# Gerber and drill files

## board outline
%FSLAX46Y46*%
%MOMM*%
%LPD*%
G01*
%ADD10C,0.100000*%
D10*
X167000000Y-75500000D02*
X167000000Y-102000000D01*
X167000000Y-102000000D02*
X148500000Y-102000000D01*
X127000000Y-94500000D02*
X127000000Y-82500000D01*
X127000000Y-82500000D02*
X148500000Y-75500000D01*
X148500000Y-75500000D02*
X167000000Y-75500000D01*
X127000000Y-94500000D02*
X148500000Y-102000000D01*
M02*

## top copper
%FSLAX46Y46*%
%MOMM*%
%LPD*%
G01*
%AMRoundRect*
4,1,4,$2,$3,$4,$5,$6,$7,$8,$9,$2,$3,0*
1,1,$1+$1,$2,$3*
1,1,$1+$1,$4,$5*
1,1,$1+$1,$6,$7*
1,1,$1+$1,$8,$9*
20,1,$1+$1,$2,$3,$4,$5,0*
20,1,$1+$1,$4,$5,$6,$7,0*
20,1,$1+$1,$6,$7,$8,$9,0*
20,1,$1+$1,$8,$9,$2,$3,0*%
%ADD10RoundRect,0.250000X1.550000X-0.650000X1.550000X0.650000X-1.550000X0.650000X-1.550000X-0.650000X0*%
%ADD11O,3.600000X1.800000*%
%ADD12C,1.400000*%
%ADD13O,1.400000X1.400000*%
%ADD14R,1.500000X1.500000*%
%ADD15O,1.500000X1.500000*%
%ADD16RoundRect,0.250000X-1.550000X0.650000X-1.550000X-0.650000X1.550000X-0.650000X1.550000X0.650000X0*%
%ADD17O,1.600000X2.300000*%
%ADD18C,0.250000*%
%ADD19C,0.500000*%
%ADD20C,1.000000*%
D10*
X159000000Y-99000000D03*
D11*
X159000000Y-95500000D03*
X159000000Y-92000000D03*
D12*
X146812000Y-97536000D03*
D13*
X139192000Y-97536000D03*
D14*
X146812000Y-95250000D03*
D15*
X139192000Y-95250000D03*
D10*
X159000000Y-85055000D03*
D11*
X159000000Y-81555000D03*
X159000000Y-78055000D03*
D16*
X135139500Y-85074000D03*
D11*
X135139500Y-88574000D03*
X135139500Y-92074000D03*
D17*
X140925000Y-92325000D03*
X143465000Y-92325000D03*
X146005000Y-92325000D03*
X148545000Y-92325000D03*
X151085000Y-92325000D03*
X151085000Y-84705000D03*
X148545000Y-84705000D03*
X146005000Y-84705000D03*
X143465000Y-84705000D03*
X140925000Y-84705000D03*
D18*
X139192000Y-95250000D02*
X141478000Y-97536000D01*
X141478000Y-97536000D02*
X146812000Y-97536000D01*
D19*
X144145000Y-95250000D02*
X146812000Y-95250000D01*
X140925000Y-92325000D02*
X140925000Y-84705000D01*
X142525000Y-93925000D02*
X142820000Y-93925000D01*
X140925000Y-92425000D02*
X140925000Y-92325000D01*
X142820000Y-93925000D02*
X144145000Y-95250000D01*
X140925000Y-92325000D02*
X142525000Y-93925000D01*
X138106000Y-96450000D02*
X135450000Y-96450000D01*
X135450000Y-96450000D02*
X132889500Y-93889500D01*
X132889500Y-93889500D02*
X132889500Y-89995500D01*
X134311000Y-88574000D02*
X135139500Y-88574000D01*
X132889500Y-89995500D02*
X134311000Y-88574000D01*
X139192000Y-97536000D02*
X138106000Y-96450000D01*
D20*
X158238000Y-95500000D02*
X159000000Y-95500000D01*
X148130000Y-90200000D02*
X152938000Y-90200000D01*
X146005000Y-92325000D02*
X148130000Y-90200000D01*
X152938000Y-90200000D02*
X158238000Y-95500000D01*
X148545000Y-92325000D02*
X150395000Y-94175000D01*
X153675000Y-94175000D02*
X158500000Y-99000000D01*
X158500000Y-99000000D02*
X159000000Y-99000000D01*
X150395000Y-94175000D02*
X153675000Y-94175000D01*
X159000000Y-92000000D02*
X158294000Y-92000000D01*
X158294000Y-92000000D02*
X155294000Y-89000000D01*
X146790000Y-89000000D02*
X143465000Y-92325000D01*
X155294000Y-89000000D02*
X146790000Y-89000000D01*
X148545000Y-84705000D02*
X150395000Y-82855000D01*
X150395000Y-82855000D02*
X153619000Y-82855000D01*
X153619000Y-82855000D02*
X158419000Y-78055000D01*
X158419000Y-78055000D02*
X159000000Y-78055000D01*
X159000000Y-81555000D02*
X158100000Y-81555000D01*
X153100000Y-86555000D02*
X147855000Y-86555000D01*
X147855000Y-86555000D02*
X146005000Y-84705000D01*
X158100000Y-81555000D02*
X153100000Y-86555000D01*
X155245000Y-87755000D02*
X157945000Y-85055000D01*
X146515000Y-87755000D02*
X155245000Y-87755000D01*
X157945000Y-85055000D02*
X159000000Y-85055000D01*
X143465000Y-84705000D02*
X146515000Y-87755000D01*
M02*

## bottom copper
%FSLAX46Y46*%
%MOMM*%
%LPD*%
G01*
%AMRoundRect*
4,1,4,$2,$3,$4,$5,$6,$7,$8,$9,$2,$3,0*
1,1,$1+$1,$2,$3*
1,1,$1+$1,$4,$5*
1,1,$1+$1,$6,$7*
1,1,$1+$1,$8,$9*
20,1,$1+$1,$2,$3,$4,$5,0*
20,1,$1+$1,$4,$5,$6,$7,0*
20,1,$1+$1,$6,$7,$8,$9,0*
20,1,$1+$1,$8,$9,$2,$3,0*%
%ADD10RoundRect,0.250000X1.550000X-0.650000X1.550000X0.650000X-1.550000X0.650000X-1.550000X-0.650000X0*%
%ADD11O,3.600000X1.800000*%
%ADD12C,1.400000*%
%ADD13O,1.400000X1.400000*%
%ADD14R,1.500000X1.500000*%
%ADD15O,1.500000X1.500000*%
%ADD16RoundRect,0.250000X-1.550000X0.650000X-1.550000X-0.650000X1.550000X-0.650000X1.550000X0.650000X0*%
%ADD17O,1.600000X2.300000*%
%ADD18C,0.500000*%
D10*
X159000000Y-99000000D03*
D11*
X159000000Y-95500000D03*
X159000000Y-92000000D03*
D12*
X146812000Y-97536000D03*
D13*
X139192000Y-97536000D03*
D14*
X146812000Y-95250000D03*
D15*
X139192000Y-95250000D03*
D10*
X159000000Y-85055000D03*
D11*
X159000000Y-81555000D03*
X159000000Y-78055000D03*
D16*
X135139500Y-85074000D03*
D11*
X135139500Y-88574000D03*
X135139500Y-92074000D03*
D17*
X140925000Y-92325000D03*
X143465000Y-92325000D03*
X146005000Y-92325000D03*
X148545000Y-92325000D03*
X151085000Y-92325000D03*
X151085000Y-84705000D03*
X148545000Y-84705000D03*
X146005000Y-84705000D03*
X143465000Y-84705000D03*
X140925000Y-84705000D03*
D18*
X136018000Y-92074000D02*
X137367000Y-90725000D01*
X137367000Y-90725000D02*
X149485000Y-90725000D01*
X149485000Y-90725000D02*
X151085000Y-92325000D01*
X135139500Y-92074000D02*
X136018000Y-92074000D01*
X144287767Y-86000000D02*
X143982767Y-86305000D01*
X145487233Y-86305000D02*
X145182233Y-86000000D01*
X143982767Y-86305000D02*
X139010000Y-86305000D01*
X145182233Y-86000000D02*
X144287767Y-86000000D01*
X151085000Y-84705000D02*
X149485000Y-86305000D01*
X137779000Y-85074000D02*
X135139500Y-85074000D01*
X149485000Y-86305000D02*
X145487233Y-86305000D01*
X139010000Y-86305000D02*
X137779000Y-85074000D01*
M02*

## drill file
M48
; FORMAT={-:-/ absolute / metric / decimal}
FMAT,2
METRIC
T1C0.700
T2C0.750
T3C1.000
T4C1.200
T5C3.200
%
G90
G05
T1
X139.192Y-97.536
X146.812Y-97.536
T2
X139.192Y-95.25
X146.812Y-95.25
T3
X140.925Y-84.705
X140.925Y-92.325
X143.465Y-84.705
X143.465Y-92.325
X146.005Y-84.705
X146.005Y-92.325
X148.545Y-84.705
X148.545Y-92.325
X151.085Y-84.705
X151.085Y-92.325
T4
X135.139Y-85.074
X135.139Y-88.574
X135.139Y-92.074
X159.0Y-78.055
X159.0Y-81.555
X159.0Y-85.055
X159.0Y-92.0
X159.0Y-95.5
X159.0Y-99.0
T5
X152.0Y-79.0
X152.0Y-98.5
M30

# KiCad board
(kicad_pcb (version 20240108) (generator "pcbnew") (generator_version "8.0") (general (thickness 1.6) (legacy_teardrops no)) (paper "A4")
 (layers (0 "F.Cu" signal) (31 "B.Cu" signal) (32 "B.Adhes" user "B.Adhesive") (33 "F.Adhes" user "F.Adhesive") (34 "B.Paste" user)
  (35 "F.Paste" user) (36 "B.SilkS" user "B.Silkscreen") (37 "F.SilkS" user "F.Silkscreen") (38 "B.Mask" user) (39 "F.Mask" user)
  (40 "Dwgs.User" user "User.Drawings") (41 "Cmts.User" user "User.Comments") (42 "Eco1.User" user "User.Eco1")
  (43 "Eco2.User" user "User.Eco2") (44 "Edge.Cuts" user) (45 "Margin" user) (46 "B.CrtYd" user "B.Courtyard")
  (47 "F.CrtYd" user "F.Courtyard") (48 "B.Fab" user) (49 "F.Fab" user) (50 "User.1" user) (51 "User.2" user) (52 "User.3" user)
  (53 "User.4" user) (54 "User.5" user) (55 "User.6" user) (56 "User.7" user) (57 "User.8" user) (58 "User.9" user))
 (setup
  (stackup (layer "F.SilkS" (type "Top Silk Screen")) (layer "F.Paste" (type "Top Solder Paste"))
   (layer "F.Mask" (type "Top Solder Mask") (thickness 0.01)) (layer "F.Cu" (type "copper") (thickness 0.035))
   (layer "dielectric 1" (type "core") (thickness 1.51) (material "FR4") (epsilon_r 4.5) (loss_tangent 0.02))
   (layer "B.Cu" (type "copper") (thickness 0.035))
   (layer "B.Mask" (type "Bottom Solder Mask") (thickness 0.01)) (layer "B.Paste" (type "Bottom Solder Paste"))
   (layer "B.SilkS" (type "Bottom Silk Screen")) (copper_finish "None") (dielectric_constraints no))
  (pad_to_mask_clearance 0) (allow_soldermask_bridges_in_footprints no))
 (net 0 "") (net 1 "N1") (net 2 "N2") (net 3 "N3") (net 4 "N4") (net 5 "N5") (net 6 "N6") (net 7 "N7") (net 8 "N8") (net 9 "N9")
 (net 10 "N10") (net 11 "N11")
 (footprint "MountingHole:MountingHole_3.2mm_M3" (layer "F.Cu") (at 152 98.5)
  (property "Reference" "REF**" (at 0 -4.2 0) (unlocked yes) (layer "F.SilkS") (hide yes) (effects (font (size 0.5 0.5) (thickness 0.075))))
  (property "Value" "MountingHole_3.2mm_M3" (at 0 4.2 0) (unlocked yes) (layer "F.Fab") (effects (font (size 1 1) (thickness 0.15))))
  (pad "" np_thru_hole circle (at 0 0) (size 3.2 3.2) (drill 3.2) (layers "*.Cu" "*.Mask")))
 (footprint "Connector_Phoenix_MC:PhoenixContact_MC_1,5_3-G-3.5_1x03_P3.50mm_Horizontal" (layer "F.Cu") (at 159 99 90)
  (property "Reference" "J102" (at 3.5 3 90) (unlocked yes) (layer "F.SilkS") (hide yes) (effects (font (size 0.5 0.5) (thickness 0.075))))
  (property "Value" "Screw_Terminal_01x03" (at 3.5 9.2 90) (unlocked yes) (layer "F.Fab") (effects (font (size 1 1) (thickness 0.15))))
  (pad "1" thru_hole roundrect (at 0 0 90) (size 1.8 3.6) (drill 1.2) (layers "*.Cu" "*.Mask") (remove_unused_layers no)
   (roundrect_rratio 0.138889) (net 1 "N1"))
  (pad "2" thru_hole oval (at 3.5 0 90) (size 1.8 3.6) (drill 1.2) (layers "*.Cu" "*.Mask") (remove_unused_layers no) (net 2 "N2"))
  (pad "3" thru_hole oval (at 7 0 90) (size 1.8 3.6) (drill 1.2) (layers "*.Cu" "*.Mask") (remove_unused_layers no) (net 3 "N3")))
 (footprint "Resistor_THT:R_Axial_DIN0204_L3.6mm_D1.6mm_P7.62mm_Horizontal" (layer "F.Cu") (at 146.812 97.536 180)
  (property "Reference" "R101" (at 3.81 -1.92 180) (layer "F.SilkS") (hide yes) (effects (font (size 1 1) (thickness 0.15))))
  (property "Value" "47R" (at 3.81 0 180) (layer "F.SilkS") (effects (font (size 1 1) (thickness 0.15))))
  (pad "1" thru_hole circle (at 0 0 180) (size 1.4 1.4) (drill 0.7) (layers "*.Cu" "*.Mask") (remove_unused_layers no) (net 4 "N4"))
  (pad "2" thru_hole oval (at 7.62 0 180) (size 1.4 1.4) (drill 0.7) (layers "*.Cu" "*.Mask") (remove_unused_layers no) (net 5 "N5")))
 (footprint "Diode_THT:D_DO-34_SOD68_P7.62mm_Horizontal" (layer "F.Cu") (at 146.812 95.25 180)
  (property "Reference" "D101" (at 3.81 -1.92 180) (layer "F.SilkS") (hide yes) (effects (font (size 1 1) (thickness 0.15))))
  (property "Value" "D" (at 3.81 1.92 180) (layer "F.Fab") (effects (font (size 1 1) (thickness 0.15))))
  (pad "1" thru_hole rect (at 0 0 180) (size 1.5 1.5) (drill 0.75) (layers "*.Cu" "*.Mask") (remove_unused_layers no) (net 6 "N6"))
  (pad "2" thru_hole oval (at 7.62 0 180) (size 1.5 1.5) (drill 0.75) (layers "*.Cu" "*.Mask") (remove_unused_layers no) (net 4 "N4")))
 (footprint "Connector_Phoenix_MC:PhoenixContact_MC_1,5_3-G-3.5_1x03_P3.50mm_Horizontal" (layer "F.Cu") (at 159 85.055 90)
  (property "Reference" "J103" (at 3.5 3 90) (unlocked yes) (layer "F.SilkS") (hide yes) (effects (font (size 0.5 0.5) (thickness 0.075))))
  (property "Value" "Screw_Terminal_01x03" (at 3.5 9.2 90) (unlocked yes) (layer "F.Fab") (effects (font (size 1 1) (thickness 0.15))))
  (pad "1" thru_hole roundrect (at 0 0 90) (size 1.8 3.6) (drill 1.2) (layers "*.Cu" "*.Mask") (remove_unused_layers no)
   (roundrect_rratio 0.138889) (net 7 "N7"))
  (pad "2" thru_hole oval (at 3.5 0 90) (size 1.8 3.6) (drill 1.2) (layers "*.Cu" "*.Mask") (remove_unused_layers no) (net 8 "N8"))
  (pad "3" thru_hole oval (at 7 0 90) (size 1.8 3.6) (drill 1.2) (layers "*.Cu" "*.Mask") (remove_unused_layers no) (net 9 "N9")))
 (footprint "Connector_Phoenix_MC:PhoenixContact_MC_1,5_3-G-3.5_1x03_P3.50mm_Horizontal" (layer "F.Cu") (at 135.1395 85.074 -90)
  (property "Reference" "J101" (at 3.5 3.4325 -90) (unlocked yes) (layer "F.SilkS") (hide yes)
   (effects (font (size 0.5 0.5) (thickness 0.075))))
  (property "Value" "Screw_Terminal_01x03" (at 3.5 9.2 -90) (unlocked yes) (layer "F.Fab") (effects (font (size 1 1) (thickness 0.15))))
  (pad "1" thru_hole roundrect (at 0 0 270) (size 1.8 3.6) (drill 1.2) (layers "*.Cu" "*.Mask") (remove_unused_layers no)
   (roundrect_rratio 0.138889) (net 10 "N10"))
  (pad "2" thru_hole oval (at 3.5 0 270) (size 1.8 3.6) (drill 1.2) (layers "*.Cu" "*.Mask") (remove_unused_layers no) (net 5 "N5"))
  (pad "3" thru_hole oval (at 7 0 270) (size 1.8 3.6) (drill 1.2) (layers "*.Cu" "*.Mask") (remove_unused_layers no) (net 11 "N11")))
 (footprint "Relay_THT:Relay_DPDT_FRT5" (layer "F.Cu") (at 140.925 92.325 90)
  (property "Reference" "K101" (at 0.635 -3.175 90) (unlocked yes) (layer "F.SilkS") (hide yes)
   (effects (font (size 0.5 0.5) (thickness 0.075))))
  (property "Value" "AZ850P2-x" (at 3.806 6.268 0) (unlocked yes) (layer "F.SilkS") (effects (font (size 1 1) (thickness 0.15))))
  (pad "1" thru_hole oval (at 0 0 90) (size 2.3 1.6) (drill 1) (layers "*.Cu" "*.Mask") (remove_unused_layers no) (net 6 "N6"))
  (pad "2" thru_hole oval (at 0 2.54 90) (size 2.3 1.6) (drill 1) (layers "*.Cu" "*.Mask") (remove_unused_layers no) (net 3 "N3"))
  (pad "3" thru_hole oval (at 0 5.08 90) (size 2.3 1.6) (drill 1) (layers "*.Cu" "*.Mask") (remove_unused_layers no) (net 2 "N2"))
  (pad "4" thru_hole oval (at 0 7.62 90) (size 2.3 1.6) (drill 1) (layers "*.Cu" "*.Mask") (remove_unused_layers no) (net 1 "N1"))
  (pad "5" thru_hole oval (at 0 10.16 90) (size 2.3 1.6) (drill 1) (layers "*.Cu" "*.Mask") (remove_unused_layers no) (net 11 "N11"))
  (pad "6" thru_hole oval (at 7.62 10.16 90) (size 2.3 1.6) (drill 1) (layers "*.Cu" "*.Mask") (remove_unused_layers no) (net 10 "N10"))
  (pad "7" thru_hole oval (at 7.62 7.62 90) (size 2.3 1.6) (drill 1) (layers "*.Cu" "*.Mask") (remove_unused_layers no) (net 9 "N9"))
  (pad "8" thru_hole oval (at 7.62 5.08 90) (size 2.3 1.6) (drill 1) (layers "*.Cu" "*.Mask") (remove_unused_layers no) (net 8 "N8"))
  (pad "9" thru_hole oval (at 7.62 2.54 90) (size 2.3 1.6) (drill 1) (layers "*.Cu" "*.Mask") (remove_unused_layers no) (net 7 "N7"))
  (pad "10" thru_hole oval (at 7.62 0 90) (size 2.3 1.6) (drill 1) (layers "*.Cu" "*.Mask") (remove_unused_layers no) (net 6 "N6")))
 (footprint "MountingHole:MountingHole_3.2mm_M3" (layer "F.Cu") (at 152 79)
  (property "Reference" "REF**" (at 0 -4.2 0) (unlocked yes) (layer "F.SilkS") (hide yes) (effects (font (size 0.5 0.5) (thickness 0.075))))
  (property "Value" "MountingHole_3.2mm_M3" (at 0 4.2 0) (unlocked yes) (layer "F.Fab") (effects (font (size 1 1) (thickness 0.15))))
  (pad "" np_thru_hole circle (at 0 0) (size 3.2 3.2) (drill 3.2) (layers "F&B.Cu" "*.Mask")))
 (gr_line (start 167 75.5) (end 167 102) (stroke (width 0.1) (type default)) (layer "Edge.Cuts"))
 (gr_line (start 167 102) (end 148.5 102) (stroke (width 0.1) (type default)) (layer "Edge.Cuts"))
 (gr_line (start 127 94.5) (end 127 82.5) (stroke (width 0.1) (type default)) (layer "Edge.Cuts"))
 (gr_line (start 127 82.5) (end 148.5 75.5) (stroke (width 0.1) (type default)) (layer "Edge.Cuts"))
 (gr_line (start 148.5 75.5) (end 167 75.5) (stroke (width 0.1) (type default)) (layer "Edge.Cuts"))
 (gr_line (start 127 94.5) (end 148.5 102) (stroke (width 0.1) (type default)) (layer "Edge.Cuts"))
 (segment (start 139.192 95.25) (end 141.478 97.536) (width 0.25) (layer "F.Cu") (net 4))
 (segment (start 141.478 97.536) (end 146.812 97.536) (width 0.25) (layer "F.Cu") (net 4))
 (segment (start 144.145 95.25) (end 146.812 95.25) (width 0.5) (layer "F.Cu") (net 6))
 (segment (start 140.925 92.325) (end 140.925 84.705) (width 0.5) (layer "F.Cu") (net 6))
 (segment (start 142.525 93.925) (end 142.82 93.925) (width 0.5) (layer "F.Cu") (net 6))
 (segment (start 140.925 92.425) (end 140.925 92.325) (width 0.5) (layer "F.Cu") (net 6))
 (segment (start 142.82 93.925) (end 144.145 95.25) (width 0.5) (layer "F.Cu") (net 6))
 (segment (start 140.925 92.325) (end 142.525 93.925) (width 0.5) (layer "F.Cu") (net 6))
 (segment (start 136.018 92.074) (end 137.367 90.725) (width 0.5) (layer "B.Cu") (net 11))
 (segment (start 137.367 90.725) (end 149.485 90.725) (width 0.5) (layer "B.Cu") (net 11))
 (segment (start 149.485 90.725) (end 151.085 92.325) (width 0.5) (layer "B.Cu") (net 11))
 (segment (start 135.1395 92.074) (end 136.018 92.074) (width 0.5) (layer "B.Cu") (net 11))
 (segment (start 144.287767 86) (end 143.982767 86.305) (width 0.5) (layer "B.Cu") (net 10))
 (segment (start 145.487233 86.305) (end 145.182233 86) (width 0.5) (layer "B.Cu") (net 10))
 (segment (start 143.982767 86.305) (end 139.01 86.305) (width 0.5) (layer "B.Cu") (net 10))
 (segment (start 145.182233 86) (end 144.287767 86) (width 0.5) (layer "B.Cu") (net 10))
 (segment (start 151.085 84.705) (end 149.485 86.305) (width 0.5) (layer "B.Cu") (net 10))
 (segment (start 137.779 85.074) (end 135.1395 85.074) (width 0.5) (layer "B.Cu") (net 10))
 (segment (start 149.485 86.305) (end 145.487233 86.305) (width 0.5) (layer "B.Cu") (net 10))
 (segment (start 139.01 86.305) (end 137.779 85.074) (width 0.5) (layer "B.Cu") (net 10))
 (segment (start 138.106 96.45) (end 135.45 96.45) (width 0.5) (layer "F.Cu") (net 5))
 (segment (start 135.45 96.45) (end 132.8895 93.8895) (width 0.5) (layer "F.Cu") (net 5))
 (segment (start 132.8895 93.8895) (end 132.8895 89.9955) (width 0.5) (layer "F.Cu") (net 5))
 (segment (start 134.311 88.574) (end 135.1395 88.574) (width 0.5) (layer "F.Cu") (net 5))
 (segment (start 132.8895 89.9955) (end 134.311 88.574) (width 0.5) (layer "F.Cu") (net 5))
 (segment (start 139.192 97.536) (end 138.106 96.45) (width 0.5) (layer "F.Cu") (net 5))
 (segment (start 158.238 95.5) (end 159 95.5) (width 1) (layer "F.Cu") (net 2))
 (segment (start 148.13 90.2) (end 152.938 90.2) (width 1) (layer "F.Cu") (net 2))
 (segment (start 146.005 92.325) (end 148.13 90.2) (width 1) (layer "F.Cu") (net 2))
 (segment (start 152.938 90.2) (end 158.238 95.5) (width 1) (layer "F.Cu") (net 2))
 (segment (start 148.545 92.325) (end 150.395 94.175) (width 1) (layer "F.Cu") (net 1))
 (segment (start 153.675 94.175) (end 158.5 99) (width 1) (layer "F.Cu") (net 1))
 (segment (start 158.5 99) (end 159 99) (width 1) (layer "F.Cu") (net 1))
 (segment (start 150.395 94.175) (end 153.675 94.175) (width 1) (layer "F.Cu") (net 1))
 (segment (start 159 92) (end 158.294 92) (width 1) (layer "F.Cu") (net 3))
 (segment (start 158.294 92) (end 155.294 89) (width 1) (layer "F.Cu") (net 3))
 (segment (start 146.79 89) (end 143.465 92.325) (width 1) (layer "F.Cu") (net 3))
 (segment (start 155.294 89) (end 146.79 89) (width 1) (layer "F.Cu") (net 3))
 (segment (start 148.545 84.705) (end 150.395 82.855) (width 1) (layer "F.Cu") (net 9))
 (segment (start 150.395 82.855) (end 153.619 82.855) (width 1) (layer "F.Cu") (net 9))
 (segment (start 153.619 82.855) (end 158.419 78.055) (width 1) (layer "F.Cu") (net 9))
 (segment (start 158.419 78.055) (end 159 78.055) (width 1) (layer "F.Cu") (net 9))
 (segment (start 159 81.555) (end 158.1 81.555) (width 1) (layer "F.Cu") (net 8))
 (segment (start 153.1 86.555) (end 147.855 86.555) (width 1) (layer "F.Cu") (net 8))
 (segment (start 147.855 86.555) (end 146.005 84.705) (width 1) (layer "F.Cu") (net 8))
 (segment (start 158.1 81.555) (end 153.1 86.555) (width 1) (layer "F.Cu") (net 8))
 (segment (start 155.245 87.755) (end 157.945 85.055) (width 1) (layer "F.Cu") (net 7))
 (segment (start 146.515 87.755) (end 155.245 87.755) (width 1) (layer "F.Cu") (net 7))
 (segment (start 157.945 85.055) (end 159 85.055) (width 1) (layer "F.Cu") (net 7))
 (segment (start 143.465 84.705) (end 146.515 87.755) (width 1) (layer "F.Cu") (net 7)))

